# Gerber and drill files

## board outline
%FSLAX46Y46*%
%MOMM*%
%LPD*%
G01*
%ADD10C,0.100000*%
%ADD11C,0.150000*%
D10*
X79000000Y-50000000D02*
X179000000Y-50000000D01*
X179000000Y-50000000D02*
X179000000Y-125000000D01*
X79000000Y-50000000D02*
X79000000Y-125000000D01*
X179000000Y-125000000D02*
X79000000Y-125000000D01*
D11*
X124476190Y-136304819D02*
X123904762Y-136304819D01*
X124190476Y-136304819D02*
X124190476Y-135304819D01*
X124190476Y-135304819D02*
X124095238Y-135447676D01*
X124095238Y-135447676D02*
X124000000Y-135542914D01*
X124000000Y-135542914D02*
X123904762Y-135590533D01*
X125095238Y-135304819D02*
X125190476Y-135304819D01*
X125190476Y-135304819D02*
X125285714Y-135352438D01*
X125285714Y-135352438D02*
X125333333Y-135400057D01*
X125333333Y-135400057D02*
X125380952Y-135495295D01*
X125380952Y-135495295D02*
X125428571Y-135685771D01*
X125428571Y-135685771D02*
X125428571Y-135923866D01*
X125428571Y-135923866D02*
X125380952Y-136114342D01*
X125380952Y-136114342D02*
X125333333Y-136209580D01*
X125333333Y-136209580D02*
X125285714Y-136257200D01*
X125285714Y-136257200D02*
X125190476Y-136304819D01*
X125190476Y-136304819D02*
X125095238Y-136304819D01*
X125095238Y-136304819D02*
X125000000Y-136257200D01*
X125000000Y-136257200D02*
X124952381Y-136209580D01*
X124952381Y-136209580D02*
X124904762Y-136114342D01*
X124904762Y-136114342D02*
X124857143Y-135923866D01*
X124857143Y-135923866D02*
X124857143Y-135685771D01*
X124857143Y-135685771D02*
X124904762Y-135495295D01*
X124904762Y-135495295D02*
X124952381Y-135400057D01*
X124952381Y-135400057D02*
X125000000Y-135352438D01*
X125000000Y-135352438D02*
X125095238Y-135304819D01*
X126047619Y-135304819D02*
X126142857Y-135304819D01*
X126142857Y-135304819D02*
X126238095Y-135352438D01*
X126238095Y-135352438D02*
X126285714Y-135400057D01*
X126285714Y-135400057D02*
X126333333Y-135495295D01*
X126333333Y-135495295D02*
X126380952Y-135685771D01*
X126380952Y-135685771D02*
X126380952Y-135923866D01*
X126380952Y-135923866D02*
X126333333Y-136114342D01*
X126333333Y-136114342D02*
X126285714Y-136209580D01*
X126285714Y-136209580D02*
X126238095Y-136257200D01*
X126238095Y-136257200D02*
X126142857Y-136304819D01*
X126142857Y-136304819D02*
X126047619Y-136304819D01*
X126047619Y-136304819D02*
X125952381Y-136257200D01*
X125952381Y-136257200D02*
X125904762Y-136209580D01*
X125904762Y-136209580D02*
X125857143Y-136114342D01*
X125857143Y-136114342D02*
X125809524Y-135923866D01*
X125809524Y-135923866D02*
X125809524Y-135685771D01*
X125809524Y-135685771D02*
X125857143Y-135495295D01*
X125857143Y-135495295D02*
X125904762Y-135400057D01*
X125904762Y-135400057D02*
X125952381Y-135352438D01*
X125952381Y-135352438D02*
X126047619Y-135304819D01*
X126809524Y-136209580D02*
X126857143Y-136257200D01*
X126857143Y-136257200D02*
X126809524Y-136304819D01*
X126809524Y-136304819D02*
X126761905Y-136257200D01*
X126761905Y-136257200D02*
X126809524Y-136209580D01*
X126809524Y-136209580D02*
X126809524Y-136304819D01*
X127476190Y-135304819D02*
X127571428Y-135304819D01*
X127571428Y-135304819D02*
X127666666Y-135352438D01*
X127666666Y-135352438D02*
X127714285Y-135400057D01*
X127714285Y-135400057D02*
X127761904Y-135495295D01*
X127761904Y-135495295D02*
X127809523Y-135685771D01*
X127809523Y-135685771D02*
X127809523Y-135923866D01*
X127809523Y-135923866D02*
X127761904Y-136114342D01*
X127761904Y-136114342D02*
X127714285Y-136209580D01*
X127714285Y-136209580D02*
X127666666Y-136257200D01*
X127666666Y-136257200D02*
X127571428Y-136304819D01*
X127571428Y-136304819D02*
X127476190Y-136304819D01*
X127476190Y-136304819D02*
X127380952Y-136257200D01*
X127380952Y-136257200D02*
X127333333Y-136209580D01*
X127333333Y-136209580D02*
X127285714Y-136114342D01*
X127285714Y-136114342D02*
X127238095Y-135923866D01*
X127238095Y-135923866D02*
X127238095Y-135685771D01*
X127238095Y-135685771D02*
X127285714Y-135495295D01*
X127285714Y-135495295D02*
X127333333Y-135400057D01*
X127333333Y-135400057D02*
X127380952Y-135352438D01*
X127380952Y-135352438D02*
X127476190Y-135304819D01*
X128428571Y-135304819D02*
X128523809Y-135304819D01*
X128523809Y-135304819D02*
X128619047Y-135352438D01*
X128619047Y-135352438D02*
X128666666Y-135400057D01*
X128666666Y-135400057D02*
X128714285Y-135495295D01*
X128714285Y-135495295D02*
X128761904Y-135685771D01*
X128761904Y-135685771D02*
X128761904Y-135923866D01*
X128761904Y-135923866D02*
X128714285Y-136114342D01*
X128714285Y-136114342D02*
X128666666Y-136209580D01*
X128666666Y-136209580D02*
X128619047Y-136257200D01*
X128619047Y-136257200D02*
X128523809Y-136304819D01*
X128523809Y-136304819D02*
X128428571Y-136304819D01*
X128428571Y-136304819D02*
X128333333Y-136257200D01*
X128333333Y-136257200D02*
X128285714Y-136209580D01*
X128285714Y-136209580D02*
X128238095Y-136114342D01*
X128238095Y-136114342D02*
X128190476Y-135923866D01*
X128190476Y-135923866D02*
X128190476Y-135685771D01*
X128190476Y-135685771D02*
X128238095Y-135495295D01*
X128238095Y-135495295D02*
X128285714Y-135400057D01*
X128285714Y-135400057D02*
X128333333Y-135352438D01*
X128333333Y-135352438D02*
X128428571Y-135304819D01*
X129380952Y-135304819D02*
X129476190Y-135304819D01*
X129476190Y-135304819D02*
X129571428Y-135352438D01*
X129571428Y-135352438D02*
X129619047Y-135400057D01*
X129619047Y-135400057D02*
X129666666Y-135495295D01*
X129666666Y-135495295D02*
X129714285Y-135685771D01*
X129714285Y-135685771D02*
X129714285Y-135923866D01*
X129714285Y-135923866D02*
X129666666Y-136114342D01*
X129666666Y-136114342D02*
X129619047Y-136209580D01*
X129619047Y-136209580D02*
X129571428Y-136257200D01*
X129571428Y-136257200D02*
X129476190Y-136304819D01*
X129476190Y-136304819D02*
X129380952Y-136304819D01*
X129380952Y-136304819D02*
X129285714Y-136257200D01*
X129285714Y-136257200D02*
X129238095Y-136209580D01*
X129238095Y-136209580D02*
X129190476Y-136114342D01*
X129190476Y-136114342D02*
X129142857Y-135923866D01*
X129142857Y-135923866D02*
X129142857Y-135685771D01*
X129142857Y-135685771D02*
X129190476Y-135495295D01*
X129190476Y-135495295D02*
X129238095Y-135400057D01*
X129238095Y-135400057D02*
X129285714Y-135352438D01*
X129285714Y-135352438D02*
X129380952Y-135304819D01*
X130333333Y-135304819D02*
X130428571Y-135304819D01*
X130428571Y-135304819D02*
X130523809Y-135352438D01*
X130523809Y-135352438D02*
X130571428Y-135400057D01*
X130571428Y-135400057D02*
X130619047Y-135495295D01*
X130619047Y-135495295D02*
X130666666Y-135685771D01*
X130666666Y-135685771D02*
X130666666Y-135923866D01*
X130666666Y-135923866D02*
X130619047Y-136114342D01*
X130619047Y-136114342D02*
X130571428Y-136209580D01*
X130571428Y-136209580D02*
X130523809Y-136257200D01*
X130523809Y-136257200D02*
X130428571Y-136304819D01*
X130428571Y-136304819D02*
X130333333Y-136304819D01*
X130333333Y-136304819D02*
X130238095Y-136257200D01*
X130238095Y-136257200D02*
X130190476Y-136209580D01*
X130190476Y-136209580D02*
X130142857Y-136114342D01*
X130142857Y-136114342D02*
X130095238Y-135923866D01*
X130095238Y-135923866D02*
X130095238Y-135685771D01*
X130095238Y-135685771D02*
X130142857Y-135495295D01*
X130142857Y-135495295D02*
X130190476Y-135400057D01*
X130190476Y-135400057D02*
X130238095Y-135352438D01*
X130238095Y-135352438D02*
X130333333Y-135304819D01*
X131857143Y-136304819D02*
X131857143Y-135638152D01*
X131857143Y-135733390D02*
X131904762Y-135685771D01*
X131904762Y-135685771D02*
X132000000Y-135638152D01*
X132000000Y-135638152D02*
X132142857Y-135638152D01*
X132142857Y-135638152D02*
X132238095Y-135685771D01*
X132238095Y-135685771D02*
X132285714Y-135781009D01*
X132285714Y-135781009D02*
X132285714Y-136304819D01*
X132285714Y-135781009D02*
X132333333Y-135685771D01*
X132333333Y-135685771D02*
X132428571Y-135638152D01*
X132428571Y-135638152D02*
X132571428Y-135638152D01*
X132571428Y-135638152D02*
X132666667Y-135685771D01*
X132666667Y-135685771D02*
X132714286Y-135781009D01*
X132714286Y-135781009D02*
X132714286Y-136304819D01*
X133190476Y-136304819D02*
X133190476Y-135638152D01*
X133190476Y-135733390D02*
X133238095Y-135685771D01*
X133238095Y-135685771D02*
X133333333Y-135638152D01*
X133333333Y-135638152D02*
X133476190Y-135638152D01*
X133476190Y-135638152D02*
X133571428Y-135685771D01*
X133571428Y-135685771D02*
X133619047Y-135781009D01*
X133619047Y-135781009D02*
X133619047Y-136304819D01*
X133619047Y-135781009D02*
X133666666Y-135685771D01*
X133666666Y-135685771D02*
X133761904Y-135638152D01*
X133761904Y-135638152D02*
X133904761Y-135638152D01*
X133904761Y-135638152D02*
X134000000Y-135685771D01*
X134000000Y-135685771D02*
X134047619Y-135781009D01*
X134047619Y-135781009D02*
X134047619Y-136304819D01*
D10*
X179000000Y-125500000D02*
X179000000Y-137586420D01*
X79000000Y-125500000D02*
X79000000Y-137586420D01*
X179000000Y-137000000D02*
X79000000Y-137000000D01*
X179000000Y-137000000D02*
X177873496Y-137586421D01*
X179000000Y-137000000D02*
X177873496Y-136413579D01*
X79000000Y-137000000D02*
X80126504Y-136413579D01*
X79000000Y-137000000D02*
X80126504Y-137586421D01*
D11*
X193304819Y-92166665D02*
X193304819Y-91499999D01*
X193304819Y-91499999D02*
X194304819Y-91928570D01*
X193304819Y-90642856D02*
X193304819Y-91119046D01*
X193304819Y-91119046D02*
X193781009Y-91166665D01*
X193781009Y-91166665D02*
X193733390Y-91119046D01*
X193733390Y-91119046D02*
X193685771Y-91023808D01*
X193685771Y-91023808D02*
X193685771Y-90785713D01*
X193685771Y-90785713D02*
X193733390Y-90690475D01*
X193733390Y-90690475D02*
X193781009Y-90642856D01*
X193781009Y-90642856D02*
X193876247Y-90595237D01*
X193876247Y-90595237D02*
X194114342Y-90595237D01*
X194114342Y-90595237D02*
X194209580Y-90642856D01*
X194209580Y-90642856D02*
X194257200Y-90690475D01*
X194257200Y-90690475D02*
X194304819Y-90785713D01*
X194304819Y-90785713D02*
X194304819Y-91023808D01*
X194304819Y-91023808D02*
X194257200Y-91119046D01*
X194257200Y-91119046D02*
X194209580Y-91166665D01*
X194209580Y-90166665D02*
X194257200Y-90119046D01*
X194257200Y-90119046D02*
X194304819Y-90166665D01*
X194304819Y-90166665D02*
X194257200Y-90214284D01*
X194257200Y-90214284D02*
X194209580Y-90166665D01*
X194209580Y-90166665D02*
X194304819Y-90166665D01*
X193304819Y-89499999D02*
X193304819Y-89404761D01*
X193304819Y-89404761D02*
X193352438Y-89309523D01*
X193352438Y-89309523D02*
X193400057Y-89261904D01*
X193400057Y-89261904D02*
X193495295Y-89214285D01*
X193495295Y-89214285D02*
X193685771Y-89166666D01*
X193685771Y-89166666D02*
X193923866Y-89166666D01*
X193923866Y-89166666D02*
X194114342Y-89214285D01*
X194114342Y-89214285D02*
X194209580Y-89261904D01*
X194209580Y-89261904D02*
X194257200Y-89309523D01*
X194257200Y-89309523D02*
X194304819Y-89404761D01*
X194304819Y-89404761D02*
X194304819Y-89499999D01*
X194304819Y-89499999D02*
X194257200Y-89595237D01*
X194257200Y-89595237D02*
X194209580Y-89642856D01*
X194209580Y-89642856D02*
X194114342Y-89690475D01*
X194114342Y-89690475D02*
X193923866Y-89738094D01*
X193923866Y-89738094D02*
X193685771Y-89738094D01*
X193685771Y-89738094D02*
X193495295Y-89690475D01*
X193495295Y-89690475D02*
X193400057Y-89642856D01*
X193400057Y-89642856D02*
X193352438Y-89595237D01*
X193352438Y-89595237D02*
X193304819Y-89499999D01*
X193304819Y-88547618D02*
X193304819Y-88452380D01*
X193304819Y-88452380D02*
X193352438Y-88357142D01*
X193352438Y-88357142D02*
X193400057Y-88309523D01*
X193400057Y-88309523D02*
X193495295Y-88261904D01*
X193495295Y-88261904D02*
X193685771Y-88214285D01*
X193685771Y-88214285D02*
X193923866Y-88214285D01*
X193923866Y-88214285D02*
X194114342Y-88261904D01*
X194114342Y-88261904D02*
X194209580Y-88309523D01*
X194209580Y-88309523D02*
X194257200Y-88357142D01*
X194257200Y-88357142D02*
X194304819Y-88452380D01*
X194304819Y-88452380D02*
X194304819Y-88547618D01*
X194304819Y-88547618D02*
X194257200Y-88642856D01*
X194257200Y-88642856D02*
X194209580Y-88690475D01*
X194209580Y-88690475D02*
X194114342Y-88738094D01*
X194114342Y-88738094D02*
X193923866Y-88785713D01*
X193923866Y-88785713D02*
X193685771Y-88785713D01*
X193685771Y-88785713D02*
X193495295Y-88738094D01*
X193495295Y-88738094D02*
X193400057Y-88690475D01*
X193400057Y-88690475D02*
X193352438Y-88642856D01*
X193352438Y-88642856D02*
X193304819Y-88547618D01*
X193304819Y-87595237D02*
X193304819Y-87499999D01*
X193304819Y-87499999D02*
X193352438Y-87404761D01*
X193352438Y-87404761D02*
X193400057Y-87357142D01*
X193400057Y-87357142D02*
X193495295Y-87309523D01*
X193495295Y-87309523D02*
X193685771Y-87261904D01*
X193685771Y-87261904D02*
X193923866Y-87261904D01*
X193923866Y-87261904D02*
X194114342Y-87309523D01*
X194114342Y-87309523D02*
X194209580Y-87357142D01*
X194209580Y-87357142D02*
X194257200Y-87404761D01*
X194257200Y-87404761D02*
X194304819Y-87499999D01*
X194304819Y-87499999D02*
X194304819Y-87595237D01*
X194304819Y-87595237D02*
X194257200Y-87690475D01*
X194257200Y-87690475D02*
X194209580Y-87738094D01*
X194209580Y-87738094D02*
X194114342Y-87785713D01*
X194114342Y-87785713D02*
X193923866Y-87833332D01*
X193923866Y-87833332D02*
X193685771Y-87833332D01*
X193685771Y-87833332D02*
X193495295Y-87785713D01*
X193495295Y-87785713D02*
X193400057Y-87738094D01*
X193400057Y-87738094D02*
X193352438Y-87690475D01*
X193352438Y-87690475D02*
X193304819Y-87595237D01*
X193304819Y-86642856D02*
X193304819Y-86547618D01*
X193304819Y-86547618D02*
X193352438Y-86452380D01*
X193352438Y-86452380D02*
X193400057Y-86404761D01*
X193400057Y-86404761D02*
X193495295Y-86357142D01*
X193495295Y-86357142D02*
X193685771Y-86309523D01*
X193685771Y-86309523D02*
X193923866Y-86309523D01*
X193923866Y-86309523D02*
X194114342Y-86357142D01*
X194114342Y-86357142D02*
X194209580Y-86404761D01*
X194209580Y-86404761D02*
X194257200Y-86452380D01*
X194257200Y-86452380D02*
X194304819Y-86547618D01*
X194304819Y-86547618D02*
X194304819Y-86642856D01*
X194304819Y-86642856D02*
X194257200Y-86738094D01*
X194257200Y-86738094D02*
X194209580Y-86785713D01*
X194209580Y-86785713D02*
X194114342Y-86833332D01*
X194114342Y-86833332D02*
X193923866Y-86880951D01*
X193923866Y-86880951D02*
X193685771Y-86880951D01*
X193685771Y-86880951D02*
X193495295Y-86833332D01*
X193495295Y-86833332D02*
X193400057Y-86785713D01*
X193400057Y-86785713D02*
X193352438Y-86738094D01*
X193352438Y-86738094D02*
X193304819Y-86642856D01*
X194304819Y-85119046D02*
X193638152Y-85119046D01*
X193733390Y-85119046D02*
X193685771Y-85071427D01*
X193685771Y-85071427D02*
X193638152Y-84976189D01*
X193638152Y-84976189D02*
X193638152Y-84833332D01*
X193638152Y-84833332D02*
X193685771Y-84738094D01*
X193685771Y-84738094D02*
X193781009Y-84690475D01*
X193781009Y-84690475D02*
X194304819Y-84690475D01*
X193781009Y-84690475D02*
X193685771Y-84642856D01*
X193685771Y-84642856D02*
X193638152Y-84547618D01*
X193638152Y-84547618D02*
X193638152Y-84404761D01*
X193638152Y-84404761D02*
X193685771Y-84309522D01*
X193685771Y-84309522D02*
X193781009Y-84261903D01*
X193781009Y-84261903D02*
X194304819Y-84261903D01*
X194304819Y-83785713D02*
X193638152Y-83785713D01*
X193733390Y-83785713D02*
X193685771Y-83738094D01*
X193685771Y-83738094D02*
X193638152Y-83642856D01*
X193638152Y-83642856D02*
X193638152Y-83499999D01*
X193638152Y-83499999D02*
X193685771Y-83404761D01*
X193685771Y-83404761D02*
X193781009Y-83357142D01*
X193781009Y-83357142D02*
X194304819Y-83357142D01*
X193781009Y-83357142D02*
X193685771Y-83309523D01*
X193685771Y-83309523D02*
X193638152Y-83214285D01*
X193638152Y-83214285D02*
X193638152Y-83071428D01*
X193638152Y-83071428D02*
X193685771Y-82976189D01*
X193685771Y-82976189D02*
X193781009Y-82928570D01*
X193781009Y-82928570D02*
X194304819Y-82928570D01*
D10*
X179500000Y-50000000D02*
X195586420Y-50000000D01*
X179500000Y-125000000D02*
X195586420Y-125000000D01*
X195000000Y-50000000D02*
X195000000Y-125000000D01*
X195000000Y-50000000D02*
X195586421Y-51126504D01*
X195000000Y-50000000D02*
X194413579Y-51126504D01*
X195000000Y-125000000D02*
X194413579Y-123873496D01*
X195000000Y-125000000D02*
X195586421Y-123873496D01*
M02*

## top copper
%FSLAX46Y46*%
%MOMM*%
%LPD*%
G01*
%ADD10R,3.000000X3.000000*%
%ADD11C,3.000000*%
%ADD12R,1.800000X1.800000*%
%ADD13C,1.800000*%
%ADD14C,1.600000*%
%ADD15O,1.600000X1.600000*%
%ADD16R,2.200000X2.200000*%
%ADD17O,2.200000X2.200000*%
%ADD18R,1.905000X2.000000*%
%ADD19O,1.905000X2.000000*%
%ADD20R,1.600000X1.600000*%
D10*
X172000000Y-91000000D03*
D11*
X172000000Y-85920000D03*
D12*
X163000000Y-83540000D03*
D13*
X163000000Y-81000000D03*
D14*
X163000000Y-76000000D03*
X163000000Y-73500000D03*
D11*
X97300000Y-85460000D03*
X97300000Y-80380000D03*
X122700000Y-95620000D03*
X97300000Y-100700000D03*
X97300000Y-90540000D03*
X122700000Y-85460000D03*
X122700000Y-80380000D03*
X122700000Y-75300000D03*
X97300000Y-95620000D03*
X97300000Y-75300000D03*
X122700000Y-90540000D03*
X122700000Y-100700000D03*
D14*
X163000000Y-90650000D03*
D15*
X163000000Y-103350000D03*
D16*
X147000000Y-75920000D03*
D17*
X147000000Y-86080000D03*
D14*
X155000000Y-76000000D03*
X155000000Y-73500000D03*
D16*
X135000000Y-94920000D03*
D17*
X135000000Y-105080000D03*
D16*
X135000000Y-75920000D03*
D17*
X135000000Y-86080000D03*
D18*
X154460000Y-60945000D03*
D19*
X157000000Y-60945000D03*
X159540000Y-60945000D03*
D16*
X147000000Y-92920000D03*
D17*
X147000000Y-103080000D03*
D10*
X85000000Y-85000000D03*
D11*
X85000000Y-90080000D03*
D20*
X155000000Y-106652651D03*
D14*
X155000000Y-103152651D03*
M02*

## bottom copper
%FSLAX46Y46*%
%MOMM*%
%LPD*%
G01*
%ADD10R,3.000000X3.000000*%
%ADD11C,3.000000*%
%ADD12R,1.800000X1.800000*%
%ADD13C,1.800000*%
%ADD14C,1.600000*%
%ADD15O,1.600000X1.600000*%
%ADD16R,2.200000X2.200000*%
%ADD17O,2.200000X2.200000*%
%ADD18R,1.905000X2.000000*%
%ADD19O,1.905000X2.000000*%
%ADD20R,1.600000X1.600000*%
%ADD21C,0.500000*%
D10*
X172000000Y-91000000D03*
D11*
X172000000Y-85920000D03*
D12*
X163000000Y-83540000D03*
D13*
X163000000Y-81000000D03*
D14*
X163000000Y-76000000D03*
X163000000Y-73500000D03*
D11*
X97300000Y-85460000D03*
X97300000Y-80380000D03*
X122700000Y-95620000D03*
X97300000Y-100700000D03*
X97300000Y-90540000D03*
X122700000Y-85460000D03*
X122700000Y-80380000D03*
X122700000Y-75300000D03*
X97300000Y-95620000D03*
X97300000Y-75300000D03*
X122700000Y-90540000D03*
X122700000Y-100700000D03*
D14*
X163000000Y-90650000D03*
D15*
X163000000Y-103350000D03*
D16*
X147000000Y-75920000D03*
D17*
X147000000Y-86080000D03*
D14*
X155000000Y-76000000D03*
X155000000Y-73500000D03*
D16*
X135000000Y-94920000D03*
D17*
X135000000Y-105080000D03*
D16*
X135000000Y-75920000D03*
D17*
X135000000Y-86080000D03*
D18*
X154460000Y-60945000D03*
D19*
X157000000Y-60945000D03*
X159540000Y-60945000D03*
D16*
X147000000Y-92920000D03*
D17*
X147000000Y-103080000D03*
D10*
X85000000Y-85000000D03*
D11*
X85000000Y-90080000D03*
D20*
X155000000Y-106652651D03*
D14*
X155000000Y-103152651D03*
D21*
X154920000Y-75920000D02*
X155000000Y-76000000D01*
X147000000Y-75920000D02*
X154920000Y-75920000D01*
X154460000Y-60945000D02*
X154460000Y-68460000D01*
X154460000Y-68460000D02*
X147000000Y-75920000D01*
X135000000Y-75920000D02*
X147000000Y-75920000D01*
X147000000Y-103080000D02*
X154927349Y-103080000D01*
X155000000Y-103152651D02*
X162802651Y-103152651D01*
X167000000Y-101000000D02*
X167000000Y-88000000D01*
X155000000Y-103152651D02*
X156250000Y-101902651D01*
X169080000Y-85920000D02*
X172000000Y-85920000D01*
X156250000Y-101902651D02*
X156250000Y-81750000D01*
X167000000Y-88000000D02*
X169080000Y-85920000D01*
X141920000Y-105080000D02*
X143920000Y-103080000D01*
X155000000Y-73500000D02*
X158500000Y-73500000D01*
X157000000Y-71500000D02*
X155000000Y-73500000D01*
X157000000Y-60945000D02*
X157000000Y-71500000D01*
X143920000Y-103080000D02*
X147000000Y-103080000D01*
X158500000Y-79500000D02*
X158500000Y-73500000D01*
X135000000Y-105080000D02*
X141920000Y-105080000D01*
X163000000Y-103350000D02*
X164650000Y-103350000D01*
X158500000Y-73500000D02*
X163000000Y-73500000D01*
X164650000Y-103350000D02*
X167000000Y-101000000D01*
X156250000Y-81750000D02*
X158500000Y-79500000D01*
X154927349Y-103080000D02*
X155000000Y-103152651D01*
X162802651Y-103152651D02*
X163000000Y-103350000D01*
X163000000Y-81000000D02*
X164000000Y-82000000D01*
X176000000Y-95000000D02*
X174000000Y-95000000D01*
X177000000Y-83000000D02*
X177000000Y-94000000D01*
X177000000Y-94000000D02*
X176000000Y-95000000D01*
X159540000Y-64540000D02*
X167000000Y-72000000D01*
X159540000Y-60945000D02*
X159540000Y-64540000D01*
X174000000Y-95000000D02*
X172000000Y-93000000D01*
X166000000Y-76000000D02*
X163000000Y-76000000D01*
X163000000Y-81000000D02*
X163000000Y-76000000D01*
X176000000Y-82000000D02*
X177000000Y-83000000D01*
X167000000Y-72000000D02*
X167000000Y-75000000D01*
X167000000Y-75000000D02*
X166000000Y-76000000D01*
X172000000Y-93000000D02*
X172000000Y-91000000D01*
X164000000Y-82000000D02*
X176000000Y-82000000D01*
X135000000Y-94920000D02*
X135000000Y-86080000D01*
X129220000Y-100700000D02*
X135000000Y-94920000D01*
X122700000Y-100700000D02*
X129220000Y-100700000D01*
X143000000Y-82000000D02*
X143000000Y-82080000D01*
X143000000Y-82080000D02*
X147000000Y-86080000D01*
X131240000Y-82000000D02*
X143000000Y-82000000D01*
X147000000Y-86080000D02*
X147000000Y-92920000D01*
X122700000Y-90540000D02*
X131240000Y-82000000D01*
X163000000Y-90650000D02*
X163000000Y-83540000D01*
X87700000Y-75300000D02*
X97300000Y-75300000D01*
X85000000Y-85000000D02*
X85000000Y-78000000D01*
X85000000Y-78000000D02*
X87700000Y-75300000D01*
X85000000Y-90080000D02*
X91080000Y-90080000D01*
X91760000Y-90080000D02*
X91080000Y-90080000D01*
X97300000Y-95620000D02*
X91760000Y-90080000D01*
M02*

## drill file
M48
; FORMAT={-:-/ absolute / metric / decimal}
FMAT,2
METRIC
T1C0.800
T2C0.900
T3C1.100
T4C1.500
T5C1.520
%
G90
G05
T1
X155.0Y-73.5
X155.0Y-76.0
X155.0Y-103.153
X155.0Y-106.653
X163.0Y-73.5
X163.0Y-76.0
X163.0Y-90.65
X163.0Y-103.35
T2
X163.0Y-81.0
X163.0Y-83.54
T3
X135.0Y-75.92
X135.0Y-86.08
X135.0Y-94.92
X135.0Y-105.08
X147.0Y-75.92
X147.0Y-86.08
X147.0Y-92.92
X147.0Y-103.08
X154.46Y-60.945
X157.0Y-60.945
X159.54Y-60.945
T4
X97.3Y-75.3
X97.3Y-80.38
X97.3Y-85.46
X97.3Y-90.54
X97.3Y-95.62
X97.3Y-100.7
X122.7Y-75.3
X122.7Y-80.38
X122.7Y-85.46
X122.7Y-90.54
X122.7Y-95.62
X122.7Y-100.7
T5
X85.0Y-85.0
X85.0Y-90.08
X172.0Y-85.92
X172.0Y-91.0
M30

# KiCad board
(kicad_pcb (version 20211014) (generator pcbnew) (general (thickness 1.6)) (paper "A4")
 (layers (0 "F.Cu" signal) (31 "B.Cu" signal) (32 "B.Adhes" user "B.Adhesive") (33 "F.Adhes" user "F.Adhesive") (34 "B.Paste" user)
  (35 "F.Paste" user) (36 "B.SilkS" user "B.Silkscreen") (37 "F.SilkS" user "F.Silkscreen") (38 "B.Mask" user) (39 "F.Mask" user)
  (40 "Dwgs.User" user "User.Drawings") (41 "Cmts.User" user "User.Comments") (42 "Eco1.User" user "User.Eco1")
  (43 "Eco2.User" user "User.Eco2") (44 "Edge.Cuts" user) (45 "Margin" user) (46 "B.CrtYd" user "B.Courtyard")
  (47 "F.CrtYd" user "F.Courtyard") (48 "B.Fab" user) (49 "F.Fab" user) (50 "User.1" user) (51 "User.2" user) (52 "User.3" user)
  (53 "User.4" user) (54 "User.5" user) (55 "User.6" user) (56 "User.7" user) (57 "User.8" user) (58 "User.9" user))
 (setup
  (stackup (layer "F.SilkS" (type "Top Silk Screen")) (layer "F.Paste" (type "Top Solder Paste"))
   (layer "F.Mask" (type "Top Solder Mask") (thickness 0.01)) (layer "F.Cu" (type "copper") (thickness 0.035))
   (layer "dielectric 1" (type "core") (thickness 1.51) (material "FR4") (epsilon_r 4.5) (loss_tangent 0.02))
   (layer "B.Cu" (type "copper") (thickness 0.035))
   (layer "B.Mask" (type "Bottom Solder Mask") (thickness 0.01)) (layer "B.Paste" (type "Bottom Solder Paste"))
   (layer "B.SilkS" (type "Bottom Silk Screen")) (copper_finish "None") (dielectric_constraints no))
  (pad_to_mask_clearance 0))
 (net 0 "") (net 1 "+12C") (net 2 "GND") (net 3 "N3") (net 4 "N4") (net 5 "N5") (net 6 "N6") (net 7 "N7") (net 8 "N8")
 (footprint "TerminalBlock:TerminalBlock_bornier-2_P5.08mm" (layer "F.Cu") (at 172 91 90)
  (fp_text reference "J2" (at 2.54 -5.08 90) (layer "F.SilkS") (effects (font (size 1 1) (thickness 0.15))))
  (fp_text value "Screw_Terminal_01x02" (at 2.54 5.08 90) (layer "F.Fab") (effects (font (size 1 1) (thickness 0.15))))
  (pad "1" thru_hole rect (at 0 0 90) (size 3 3) (drill 1.52) (layers *.Cu *.Mask) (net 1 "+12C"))
  (pad "2" thru_hole circle (at 5.08 0 90) (size 3 3) (drill 1.52) (layers *.Cu *.Mask) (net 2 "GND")))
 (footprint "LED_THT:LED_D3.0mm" (layer "F.Cu") (at 163 83.54 90)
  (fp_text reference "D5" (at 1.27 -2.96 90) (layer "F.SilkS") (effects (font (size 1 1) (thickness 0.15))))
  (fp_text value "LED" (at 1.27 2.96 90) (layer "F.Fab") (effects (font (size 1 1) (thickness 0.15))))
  (pad "1" thru_hole rect (at 0 0 90) (size 1.8 1.8) (drill 0.9) (layers *.Cu *.Mask) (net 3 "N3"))
  (pad "2" thru_hole circle (at 2.54 0 90) (size 1.8 1.8) (drill 0.9) (layers *.Cu *.Mask) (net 1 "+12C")))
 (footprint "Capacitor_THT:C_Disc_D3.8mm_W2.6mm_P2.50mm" (layer "F.Cu") (at 163 76 90)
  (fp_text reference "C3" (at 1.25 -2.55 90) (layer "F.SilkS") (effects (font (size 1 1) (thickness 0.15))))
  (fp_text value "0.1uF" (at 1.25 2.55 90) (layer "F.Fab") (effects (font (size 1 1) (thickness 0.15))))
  (pad "1" thru_hole circle (at 0 0 90) (size 1.6 1.6) (drill 0.8) (layers *.Cu *.Mask) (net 1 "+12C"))
  (pad "2" thru_hole circle (at 2.5 0 90) (size 1.6 1.6) (drill 0.8) (layers *.Cu *.Mask) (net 2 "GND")))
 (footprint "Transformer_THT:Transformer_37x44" (layer "F.Cu") (at 97.3 95.62 90)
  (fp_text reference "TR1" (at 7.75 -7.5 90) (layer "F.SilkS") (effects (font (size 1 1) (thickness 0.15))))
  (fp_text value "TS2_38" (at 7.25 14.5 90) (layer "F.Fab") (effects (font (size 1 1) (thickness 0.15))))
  (pad "" thru_hole circle (at 10.16 0 90) (size 3 3) (drill 1.5) (layers *.Cu *.Mask))
  (pad "" thru_hole circle (at 15.24 0 90) (size 3 3) (drill 1.5) (layers *.Cu *.Mask))
  (pad "" thru_hole circle (at 0 25.4 90) (size 3 3) (drill 1.5) (layers *.Cu *.Mask))
  (pad "" thru_hole circle (at -5.08 0 90) (size 3 3) (drill 1.5) (layers *.Cu *.Mask))
  (pad "" thru_hole circle (at 5.08 0 90) (size 3 3) (drill 1.5) (layers *.Cu *.Mask))
  (pad "" thru_hole circle (at 10.16 25.4 90) (size 3 3) (drill 1.5) (layers *.Cu *.Mask))
  (pad "" thru_hole circle (at 15.24 25.4 90) (size 3 3) (drill 1.5) (layers *.Cu *.Mask))
  (pad "" thru_hole circle (at 20.32 25.4 90) (size 3 3) (drill 1.5) (layers *.Cu *.Mask))
  (pad "1" thru_hole circle (at 0 0 90) (size 3 3) (drill 1.5) (layers *.Cu *.Mask) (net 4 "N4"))
  (pad "2" thru_hole circle (at 20.32 0 90) (size 3 3) (drill 1.5) (layers *.Cu *.Mask) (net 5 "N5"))
  (pad "3" thru_hole circle (at 5.08 25.4 90) (size 3 3) (drill 1.5) (layers *.Cu *.Mask) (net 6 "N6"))
  (pad "4" thru_hole circle (at -5.08 25.4 90) (size 3 3) (drill 1.5) (layers *.Cu *.Mask) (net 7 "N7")))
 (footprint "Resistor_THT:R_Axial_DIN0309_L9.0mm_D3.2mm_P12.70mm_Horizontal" (layer "F.Cu") (at 163 90.65 -90)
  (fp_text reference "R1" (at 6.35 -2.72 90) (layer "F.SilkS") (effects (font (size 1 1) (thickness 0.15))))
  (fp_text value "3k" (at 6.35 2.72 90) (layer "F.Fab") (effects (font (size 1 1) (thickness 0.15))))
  (pad "1" thru_hole circle (at 0 0 270) (size 1.6 1.6) (drill 0.8) (layers *.Cu *.Mask) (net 3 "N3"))
  (pad "2" thru_hole oval (at 12.7 0 270) (size 1.6 1.6) (drill 0.8) (layers *.Cu *.Mask) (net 2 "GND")))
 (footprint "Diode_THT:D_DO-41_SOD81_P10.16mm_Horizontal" (layer "F.Cu") (at 147 75.92 -90)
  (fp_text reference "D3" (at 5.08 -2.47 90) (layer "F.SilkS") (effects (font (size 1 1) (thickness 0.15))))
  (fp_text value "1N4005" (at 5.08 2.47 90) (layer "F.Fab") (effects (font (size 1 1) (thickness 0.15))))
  (pad "1" thru_hole rect (at 0 0 270) (size 2.2 2.2) (drill 1.1) (layers *.Cu *.Mask) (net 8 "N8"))
  (pad "2" thru_hole oval (at 10.16 0 270) (size 2.2 2.2) (drill 1.1) (layers *.Cu *.Mask) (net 6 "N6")))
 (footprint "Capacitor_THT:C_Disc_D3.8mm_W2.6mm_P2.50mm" (layer "F.Cu") (at 155 76 90)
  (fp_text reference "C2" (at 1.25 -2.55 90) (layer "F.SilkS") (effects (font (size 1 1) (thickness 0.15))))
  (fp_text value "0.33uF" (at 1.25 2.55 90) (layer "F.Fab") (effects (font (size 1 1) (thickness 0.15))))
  (pad "1" thru_hole circle (at 0 0 90) (size 1.6 1.6) (drill 0.8) (layers *.Cu *.Mask) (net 8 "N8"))
  (pad "2" thru_hole circle (at 2.5 0 90) (size 1.6 1.6) (drill 0.8) (layers *.Cu *.Mask) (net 2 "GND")))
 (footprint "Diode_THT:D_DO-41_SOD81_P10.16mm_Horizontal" (layer "F.Cu") (at 135 94.92 -90)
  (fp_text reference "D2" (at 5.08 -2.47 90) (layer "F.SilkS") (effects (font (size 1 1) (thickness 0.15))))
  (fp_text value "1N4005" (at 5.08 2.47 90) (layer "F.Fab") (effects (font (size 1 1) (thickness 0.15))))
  (pad "1" thru_hole rect (at 0 0 270) (size 2.2 2.2) (drill 1.1) (layers *.Cu *.Mask) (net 7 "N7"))
  (pad "2" thru_hole oval (at 10.16 0 270) (size 2.2 2.2) (drill 1.1) (layers *.Cu *.Mask) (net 2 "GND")))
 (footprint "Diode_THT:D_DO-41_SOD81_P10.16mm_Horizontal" (layer "F.Cu") (at 135 75.92 -90)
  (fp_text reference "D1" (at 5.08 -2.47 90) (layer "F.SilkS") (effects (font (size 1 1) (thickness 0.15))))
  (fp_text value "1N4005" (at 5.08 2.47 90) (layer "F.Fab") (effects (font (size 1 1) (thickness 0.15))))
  (pad "1" thru_hole rect (at 0 0 270) (size 2.2 2.2) (drill 1.1) (layers *.Cu *.Mask) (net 8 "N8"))
  (pad "2" thru_hole oval (at 10.16 0 270) (size 2.2 2.2) (drill 1.1) (layers *.Cu *.Mask) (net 7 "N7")))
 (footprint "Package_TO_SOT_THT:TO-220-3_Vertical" (layer "F.Cu") (at 154.46 60.945)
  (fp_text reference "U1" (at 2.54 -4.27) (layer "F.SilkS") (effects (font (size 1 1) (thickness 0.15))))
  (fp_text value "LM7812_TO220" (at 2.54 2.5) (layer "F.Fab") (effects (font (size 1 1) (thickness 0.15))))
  (pad "1" thru_hole rect (at 0 0) (size 1.905 2) (drill 1.1) (layers *.Cu *.Mask) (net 8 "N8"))
  (pad "2" thru_hole oval (at 2.54 0) (size 1.905 2) (drill 1.1) (layers *.Cu *.Mask) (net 2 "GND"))
  (pad "3" thru_hole oval (at 5.08 0) (size 1.905 2) (drill 1.1) (layers *.Cu *.Mask) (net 1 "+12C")))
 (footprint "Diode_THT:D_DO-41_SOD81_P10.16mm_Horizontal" (layer "F.Cu") (at 147 92.92 -90)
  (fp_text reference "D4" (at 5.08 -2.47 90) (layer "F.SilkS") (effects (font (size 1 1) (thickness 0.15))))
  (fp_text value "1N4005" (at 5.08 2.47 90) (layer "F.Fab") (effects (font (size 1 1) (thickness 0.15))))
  (pad "1" thru_hole rect (at 0 0 270) (size 2.2 2.2) (drill 1.1) (layers *.Cu *.Mask) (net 6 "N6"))
  (pad "2" thru_hole oval (at 10.16 0 270) (size 2.2 2.2) (drill 1.1) (layers *.Cu *.Mask) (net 2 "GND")))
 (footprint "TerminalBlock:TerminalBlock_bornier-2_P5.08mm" (layer "F.Cu") (at 85 85 -90)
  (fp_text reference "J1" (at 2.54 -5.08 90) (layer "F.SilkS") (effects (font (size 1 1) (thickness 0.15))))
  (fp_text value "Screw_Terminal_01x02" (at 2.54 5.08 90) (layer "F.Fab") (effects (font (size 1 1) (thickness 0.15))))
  (pad "1" thru_hole rect (at 0 0 270) (size 3 3) (drill 1.52) (layers *.Cu *.Mask) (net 5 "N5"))
  (pad "2" thru_hole circle (at 5.08 0 270) (size 3 3) (drill 1.52) (layers *.Cu *.Mask) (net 4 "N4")))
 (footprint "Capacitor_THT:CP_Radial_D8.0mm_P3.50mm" (layer "F.Cu") (at 155 106.652651 90)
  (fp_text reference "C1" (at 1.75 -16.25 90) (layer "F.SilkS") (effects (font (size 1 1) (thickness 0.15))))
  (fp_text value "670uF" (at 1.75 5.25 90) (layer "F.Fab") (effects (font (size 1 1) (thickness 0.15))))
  (pad "1" thru_hole rect (at 0 0 90) (size 1.6 1.6) (drill 0.8) (layers *.Cu *.Mask) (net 8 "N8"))
  (pad "2" thru_hole circle (at 3.5 0 90) (size 1.6 1.6) (drill 0.8) (layers *.Cu *.Mask) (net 2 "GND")))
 (gr_line (start 79 50) (end 179 50) (layer "Edge.Cuts") (width 0.1))
 (gr_line (start 179 50) (end 179 125) (layer "Edge.Cuts") (width 0.1))
 (gr_line (start 79 50) (end 79 125) (layer "Edge.Cuts") (width 0.1))
 (gr_line (start 179 125) (end 79 125) (layer "Edge.Cuts") (width 0.1))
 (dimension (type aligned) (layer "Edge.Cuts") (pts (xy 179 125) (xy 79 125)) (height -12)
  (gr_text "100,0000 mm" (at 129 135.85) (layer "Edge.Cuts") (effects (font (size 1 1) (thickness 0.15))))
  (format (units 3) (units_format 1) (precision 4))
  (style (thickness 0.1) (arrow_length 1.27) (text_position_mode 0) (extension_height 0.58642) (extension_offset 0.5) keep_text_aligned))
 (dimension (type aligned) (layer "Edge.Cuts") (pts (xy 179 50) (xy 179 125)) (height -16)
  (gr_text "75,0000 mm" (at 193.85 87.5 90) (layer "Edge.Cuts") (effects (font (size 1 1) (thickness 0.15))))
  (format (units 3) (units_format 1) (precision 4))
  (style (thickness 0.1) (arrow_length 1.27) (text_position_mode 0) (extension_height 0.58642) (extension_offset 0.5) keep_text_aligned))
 (segment (start 154.92 75.92) (end 155 76) (width 0.5) (layer "B.Cu") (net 8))
 (segment (start 147 75.92) (end 154.92 75.92) (width 0.5) (layer "B.Cu") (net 8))
 (segment (start 154.46 60.945) (end 154.46 68.46) (width 0.5) (layer "B.Cu") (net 8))
 (segment (start 154.46 68.46) (end 147 75.92) (width 0.5) (layer "B.Cu") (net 8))
 (segment (start 135 75.92) (end 147 75.92) (width 0.5) (layer "B.Cu") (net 8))
 (segment (start 147 103.08) (end 154.927349 103.08) (width 0.5) (layer "B.Cu") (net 2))
 (segment (start 155 103.152651) (end 162.802651 103.152651) (width 0.5) (layer "B.Cu") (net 2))
 (segment (start 167 101) (end 167 88) (width 0.5) (layer "B.Cu") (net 2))
 (segment (start 155 103.152651) (end 156.25 101.902651) (width 0.5) (layer "B.Cu") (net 2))
 (segment (start 169.08 85.92) (end 172 85.92) (width 0.5) (layer "B.Cu") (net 2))
 (segment (start 156.25 101.902651) (end 156.25 81.75) (width 0.5) (layer "B.Cu") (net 2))
 (segment (start 167 88) (end 169.08 85.92) (width 0.5) (layer "B.Cu") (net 2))
 (segment (start 141.92 105.08) (end 143.92 103.08) (width 0.5) (layer "B.Cu") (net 2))
 (segment (start 155 73.5) (end 158.5 73.5) (width 0.5) (layer "B.Cu") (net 2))
 (segment (start 157 71.5) (end 155 73.5) (width 0.5) (layer "B.Cu") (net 2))
 (segment (start 157 60.945) (end 157 71.5) (width 0.5) (layer "B.Cu") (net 2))
 (segment (start 143.92 103.08) (end 147 103.08) (width 0.5) (layer "B.Cu") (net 2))
 (segment (start 158.5 79.5) (end 158.5 73.5) (width 0.5) (layer "B.Cu") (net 2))
 (segment (start 135 105.08) (end 141.92 105.08) (width 0.5) (layer "B.Cu") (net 2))
 (segment (start 163 103.35) (end 164.65 103.35) (width 0.5) (layer "B.Cu") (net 2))
 (segment (start 158.5 73.5) (end 163 73.5) (width 0.5) (layer "B.Cu") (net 2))
 (segment (start 164.65 103.35) (end 167 101) (width 0.5) (layer "B.Cu") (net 2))
 (segment (start 156.25 81.75) (end 158.5 79.5) (width 0.5) (layer "B.Cu") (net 2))
 (segment (start 154.927349 103.08) (end 155 103.152651) (width 0.5) (layer "B.Cu") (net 2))
 (segment (start 162.802651 103.152651) (end 163 103.35) (width 0.5) (layer "B.Cu") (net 2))
 (segment (start 163 81) (end 164 82) (width 0.5) (layer "B.Cu") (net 1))
 (segment (start 176 95) (end 174 95) (width 0.5) (layer "B.Cu") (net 1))
 (segment (start 177 83) (end 177 94) (width 0.5) (layer "B.Cu") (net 1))
 (segment (start 177 94) (end 176 95) (width 0.5) (layer "B.Cu") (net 1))
 (segment (start 159.54 64.54) (end 167 72) (width 0.5) (layer "B.Cu") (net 1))
 (segment (start 159.54 60.945) (end 159.54 64.54) (width 0.5) (layer "B.Cu") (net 1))
 (segment (start 174 95) (end 172 93) (width 0.5) (layer "B.Cu") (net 1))
 (segment (start 166 76) (end 163 76) (width 0.5) (layer "B.Cu") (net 1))
 (segment (start 163 81) (end 163 76) (width 0.5) (layer "B.Cu") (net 1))
 (segment (start 176 82) (end 177 83) (width 0.5) (layer "B.Cu") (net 1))
 (segment (start 167 72) (end 167 75) (width 0.5) (layer "B.Cu") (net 1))
 (segment (start 167 75) (end 166 76) (width 0.5) (layer "B.Cu") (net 1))
 (segment (start 172 93) (end 172 91) (width 0.5) (layer "B.Cu") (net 1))
 (segment (start 164 82) (end 176 82) (width 0.5) (layer "B.Cu") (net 1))
 (segment (start 135 94.92) (end 135 86.08) (width 0.5) (layer "B.Cu") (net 7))
 (segment (start 129.22 100.7) (end 135 94.92) (width 0.5) (layer "B.Cu") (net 7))
 (segment (start 122.7 100.7) (end 129.22 100.7) (width 0.5) (layer "B.Cu") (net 7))
 (segment (start 143 82) (end 143 82.08) (width 0.5) (layer "B.Cu") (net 6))
 (segment (start 143 82.08) (end 147 86.08) (width 0.5) (layer "B.Cu") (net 6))
 (segment (start 131.24 82) (end 143 82) (width 0.5) (layer "B.Cu") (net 6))
 (segment (start 147 86.08) (end 147 92.92) (width 0.5) (layer "B.Cu") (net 6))
 (segment (start 122.7 90.54) (end 131.24 82) (width 0.5) (layer "B.Cu") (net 6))
 (segment (start 163 90.65) (end 163 83.54) (width 0.5) (layer "B.Cu") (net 3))
 (segment (start 87.7 75.3) (end 97.3 75.3) (width 0.5) (layer "B.Cu") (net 5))
 (segment (start 85 85) (end 85 78) (width 0.5) (layer "B.Cu") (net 5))
 (segment (start 85 78) (end 87.7 75.3) (width 0.5) (layer "B.Cu") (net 5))
 (segment (start 85 90.08) (end 91.08 90.08) (width 0.5) (layer "B.Cu") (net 4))
 (segment (start 91.76 90.08) (end 91.08 90.08) (width 0.5) (layer "B.Cu") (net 4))
 (segment (start 97.3 95.62) (end 91.76 90.08) (width 0.5) (layer "B.Cu") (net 4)))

